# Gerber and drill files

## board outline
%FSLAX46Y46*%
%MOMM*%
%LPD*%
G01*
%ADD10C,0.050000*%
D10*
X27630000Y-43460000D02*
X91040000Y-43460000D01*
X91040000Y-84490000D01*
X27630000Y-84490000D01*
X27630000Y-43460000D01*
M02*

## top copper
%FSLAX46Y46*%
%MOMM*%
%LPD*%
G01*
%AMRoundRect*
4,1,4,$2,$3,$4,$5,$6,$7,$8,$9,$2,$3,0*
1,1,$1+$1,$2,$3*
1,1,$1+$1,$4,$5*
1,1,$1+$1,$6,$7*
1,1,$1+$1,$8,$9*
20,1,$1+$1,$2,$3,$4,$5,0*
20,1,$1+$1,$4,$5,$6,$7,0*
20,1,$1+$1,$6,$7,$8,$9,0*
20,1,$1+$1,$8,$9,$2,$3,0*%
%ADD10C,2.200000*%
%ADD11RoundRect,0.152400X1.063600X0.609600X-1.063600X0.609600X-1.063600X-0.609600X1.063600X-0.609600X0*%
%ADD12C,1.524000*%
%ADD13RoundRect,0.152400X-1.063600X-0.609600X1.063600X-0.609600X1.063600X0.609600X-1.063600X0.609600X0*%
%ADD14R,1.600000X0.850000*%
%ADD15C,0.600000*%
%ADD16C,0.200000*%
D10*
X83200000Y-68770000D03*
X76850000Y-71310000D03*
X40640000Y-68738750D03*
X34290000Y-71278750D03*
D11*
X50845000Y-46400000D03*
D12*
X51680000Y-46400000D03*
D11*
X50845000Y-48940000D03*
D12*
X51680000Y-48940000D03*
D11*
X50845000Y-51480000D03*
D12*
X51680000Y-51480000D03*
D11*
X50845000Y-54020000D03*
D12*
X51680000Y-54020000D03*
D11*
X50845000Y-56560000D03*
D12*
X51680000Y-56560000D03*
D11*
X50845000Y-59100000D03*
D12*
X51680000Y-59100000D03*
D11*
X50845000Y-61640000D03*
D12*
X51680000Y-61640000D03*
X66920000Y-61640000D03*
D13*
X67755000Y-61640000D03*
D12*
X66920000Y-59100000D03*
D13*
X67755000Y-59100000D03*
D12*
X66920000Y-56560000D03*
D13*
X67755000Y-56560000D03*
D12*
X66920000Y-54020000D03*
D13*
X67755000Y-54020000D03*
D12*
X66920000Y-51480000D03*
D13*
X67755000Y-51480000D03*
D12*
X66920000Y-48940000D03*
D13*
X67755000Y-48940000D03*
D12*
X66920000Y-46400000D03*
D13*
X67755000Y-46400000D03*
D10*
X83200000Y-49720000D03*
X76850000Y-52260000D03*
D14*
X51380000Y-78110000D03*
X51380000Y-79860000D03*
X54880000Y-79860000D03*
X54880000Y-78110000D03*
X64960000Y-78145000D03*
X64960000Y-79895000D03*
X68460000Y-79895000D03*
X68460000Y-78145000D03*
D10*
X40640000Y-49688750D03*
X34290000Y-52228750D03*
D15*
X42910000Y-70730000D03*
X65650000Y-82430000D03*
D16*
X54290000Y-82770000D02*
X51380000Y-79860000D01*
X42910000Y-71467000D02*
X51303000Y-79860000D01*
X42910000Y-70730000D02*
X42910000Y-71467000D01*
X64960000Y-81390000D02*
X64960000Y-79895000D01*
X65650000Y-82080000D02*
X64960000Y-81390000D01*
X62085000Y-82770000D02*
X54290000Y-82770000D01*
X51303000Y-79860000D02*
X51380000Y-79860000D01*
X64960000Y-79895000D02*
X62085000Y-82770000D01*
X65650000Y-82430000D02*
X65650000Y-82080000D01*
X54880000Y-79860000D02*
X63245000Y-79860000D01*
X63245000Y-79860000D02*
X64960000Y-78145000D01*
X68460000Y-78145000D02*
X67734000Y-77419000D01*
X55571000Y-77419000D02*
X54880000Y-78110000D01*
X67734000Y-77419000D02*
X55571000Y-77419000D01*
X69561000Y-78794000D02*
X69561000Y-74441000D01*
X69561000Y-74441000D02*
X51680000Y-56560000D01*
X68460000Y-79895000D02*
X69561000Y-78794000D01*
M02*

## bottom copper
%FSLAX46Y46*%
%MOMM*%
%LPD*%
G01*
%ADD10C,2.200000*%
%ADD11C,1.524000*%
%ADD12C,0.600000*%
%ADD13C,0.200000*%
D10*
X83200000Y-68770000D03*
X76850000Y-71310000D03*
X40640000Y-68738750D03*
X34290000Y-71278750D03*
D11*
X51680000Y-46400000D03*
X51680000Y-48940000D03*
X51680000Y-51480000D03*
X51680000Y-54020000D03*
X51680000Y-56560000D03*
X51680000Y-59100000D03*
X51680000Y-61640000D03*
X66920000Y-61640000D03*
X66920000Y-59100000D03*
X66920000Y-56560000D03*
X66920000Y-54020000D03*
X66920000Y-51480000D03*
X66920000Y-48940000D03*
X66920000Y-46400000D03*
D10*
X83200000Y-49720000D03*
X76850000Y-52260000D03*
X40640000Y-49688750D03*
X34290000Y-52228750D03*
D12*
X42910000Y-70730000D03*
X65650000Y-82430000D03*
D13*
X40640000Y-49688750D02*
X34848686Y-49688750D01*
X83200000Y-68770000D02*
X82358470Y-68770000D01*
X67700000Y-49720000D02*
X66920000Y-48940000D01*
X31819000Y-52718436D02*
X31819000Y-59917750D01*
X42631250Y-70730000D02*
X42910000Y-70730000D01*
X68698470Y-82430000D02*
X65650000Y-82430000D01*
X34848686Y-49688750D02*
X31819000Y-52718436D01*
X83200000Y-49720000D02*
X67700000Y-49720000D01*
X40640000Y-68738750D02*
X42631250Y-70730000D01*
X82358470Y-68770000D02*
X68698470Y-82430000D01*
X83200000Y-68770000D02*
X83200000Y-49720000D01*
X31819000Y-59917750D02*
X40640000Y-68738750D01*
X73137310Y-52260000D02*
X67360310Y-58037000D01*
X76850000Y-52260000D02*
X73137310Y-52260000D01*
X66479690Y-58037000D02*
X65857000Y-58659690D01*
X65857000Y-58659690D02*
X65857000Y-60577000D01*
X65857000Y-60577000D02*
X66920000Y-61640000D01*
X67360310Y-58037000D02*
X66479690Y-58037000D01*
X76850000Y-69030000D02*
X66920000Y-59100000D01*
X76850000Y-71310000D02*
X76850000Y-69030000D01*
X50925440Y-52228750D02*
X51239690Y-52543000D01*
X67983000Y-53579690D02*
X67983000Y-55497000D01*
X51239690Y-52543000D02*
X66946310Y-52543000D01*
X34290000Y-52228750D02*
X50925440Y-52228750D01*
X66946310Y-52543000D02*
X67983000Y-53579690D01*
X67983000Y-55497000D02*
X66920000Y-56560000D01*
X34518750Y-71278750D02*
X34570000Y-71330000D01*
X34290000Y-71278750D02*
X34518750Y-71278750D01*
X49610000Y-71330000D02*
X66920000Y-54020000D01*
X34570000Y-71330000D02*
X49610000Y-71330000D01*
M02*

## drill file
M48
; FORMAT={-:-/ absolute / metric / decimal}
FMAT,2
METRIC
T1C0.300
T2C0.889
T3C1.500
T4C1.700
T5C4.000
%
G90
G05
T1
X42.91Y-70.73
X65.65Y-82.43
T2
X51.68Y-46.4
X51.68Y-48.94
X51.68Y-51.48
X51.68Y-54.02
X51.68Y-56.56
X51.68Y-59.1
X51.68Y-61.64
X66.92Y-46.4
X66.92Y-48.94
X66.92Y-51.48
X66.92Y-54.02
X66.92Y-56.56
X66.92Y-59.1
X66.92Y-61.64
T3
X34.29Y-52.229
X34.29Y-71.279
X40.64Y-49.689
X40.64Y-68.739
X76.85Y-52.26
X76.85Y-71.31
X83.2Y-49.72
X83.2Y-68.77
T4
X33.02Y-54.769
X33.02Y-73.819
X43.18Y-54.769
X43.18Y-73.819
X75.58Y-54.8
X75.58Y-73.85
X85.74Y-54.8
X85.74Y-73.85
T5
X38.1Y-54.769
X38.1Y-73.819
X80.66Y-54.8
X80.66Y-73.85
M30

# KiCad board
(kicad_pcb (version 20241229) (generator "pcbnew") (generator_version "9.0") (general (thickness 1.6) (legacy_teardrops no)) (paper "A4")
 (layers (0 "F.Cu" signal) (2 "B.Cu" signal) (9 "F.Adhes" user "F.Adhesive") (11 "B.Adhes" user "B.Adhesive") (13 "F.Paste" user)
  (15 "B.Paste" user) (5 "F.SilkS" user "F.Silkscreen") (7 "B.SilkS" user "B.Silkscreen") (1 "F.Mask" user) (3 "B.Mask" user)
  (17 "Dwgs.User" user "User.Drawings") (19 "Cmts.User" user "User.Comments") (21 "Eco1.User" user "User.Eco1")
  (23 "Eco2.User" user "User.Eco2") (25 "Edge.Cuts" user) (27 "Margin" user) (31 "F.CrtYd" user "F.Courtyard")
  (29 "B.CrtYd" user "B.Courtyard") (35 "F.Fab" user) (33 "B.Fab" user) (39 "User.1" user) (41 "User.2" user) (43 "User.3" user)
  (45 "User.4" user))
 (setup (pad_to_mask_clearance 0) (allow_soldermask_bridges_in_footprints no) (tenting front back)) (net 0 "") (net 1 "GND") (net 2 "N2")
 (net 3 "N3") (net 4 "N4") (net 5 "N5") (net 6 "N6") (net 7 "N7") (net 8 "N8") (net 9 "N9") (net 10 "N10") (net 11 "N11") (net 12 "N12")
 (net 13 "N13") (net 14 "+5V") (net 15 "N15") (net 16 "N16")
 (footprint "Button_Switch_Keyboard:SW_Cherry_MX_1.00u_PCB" (layer "F.Cu") (at 83.2 68.77)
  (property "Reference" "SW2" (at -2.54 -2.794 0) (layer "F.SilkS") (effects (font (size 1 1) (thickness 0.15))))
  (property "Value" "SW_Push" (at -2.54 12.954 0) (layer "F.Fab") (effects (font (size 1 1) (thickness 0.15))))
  (pad "" np_thru_hole circle (at -7.62 5.08) (size 1.7 1.7) (drill 1.7) (layers "*.Cu" "*.Mask"))
  (pad "" np_thru_hole circle (at -2.54 5.08) (size 4 4) (drill 4) (layers "*.Cu" "*.Mask"))
  (pad "" np_thru_hole circle (at 2.54 5.08) (size 1.7 1.7) (drill 1.7) (layers "*.Cu" "*.Mask"))
  (pad "1" thru_hole circle (at 0 0) (size 2.2 2.2) (drill 1.5) (layers "*.Cu" "*.Mask") (remove_unused_layers no) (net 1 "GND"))
  (pad "2" thru_hole circle (at -6.35 2.54) (size 2.2 2.2) (drill 1.5) (layers "*.Cu" "*.Mask") (remove_unused_layers no) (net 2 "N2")))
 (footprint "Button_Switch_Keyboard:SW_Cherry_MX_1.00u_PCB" (layer "F.Cu") (at 40.64 68.73875)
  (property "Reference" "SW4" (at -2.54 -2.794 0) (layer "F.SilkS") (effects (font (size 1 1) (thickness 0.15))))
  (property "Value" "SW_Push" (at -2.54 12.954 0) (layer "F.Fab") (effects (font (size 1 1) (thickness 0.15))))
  (pad "" np_thru_hole circle (at -7.62 5.08) (size 1.7 1.7) (drill 1.7) (layers "*.Cu" "*.Mask"))
  (pad "" np_thru_hole circle (at -2.54 5.08) (size 4 4) (drill 4) (layers "*.Cu" "*.Mask"))
  (pad "" np_thru_hole circle (at 2.54 5.08) (size 1.7 1.7) (drill 1.7) (layers "*.Cu" "*.Mask"))
  (pad "1" thru_hole circle (at 0 0) (size 2.2 2.2) (drill 1.5) (layers "*.Cu" "*.Mask") (remove_unused_layers no) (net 1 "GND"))
  (pad "2" thru_hole circle (at -6.35 2.54) (size 2.2 2.2) (drill 1.5) (layers "*.Cu" "*.Mask") (remove_unused_layers no) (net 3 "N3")))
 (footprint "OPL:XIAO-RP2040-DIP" (layer "F.Cu") (at 59.3 54.02)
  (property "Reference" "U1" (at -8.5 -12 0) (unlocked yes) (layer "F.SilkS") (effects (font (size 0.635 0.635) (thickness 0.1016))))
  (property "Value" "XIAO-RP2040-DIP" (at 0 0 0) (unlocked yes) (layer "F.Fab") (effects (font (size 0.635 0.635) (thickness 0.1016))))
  (pad "1" smd roundrect (at -8.455 -7.62 180) (size 2.432 1.524) (layers "F.Cu" "F.Mask") (roundrect_rratio 0.1) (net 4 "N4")
   (thermal_bridge_angle 45))
  (pad "1" thru_hole circle (at -7.62 -7.62 180) (size 1.524 1.524) (drill 0.889) (layers "*.Cu" "*.Mask") (remove_unused_layers no)
   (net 4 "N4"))
  (pad "2" smd roundrect (at -8.455 -5.08 180) (size 2.432 1.524) (layers "F.Cu" "F.Mask") (roundrect_rratio 0.1) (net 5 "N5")
   (thermal_bridge_angle 45))
  (pad "2" thru_hole circle (at -7.62 -5.08 180) (size 1.524 1.524) (drill 0.889) (layers "*.Cu" "*.Mask") (remove_unused_layers no)
   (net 5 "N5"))
  (pad "3" smd roundrect (at -8.455 -2.54 180) (size 2.432 1.524) (layers "F.Cu" "F.Mask") (roundrect_rratio 0.1) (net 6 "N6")
   (thermal_bridge_angle 45))
  (pad "3" thru_hole circle (at -7.62 -2.54 180) (size 1.524 1.524) (drill 0.889) (layers "*.Cu" "*.Mask") (remove_unused_layers no)
   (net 6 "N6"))
  (pad "4" smd roundrect (at -8.455 0 180) (size 2.432 1.524) (layers "F.Cu" "F.Mask") (roundrect_rratio 0.1) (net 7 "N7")
   (thermal_bridge_angle 45))
  (pad "4" thru_hole circle (at -7.62 0 180) (size 1.524 1.524) (drill 0.889) (layers "*.Cu" "*.Mask") (remove_unused_layers no)
   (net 7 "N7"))
  (pad "5" smd roundrect (at -8.455 2.54 180) (size 2.432 1.524) (layers "F.Cu" "F.Mask") (roundrect_rratio 0.1) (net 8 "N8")
   (thermal_bridge_angle 45))
  (pad "5" thru_hole circle (at -7.62 2.54 180) (size 1.524 1.524) (drill 0.889) (layers "*.Cu" "*.Mask") (remove_unused_layers no)
   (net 8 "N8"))
  (pad "6" smd roundrect (at -8.455 5.08 180) (size 2.432 1.524) (layers "F.Cu" "F.Mask") (roundrect_rratio 0.1) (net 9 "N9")
   (thermal_bridge_angle 45))
  (pad "6" thru_hole circle (at -7.62 5.08 180) (size 1.524 1.524) (drill 0.889) (layers "*.Cu" "*.Mask") (remove_unused_layers no)
   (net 9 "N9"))
  (pad "7" smd roundrect (at -8.455 7.62 180) (size 2.432 1.524) (layers "F.Cu" "F.Mask") (roundrect_rratio 0.1) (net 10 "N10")
   (thermal_bridge_angle 45))
  (pad "7" thru_hole circle (at -7.62 7.62 180) (size 1.524 1.524) (drill 0.889) (layers "*.Cu" "*.Mask") (remove_unused_layers no)
   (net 10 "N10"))
  (pad "8" thru_hole circle (at 7.62 7.62) (size 1.524 1.524) (drill 0.889) (layers "*.Cu" "*.Mask") (remove_unused_layers no)
   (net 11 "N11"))
  (pad "8" smd roundrect (at 8.455 7.62) (size 2.432 1.524) (layers "F.Cu" "F.Mask") (roundrect_rratio 0.1) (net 11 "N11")
   (thermal_bridge_angle 45))
  (pad "9" thru_hole circle (at 7.62 5.08) (size 1.524 1.524) (drill 0.889) (layers "*.Cu" "*.Mask") (remove_unused_layers no) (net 2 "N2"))
  (pad "9" smd roundrect (at 8.455 5.08) (size 2.432 1.524) (layers "F.Cu" "F.Mask") (roundrect_rratio 0.1) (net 2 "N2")
   (thermal_bridge_angle 45))
  (pad "10" thru_hole circle (at 7.62 2.54) (size 1.524 1.524) (drill 0.889) (layers "*.Cu" "*.Mask") (remove_unused_layers no)
   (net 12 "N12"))
  (pad "10" smd roundrect (at 8.455 2.54) (size 2.432 1.524) (layers "F.Cu" "F.Mask") (roundrect_rratio 0.1) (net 12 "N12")
   (thermal_bridge_angle 45))
  (pad "11" thru_hole circle (at 7.62 0) (size 1.524 1.524) (drill 0.889) (layers "*.Cu" "*.Mask") (remove_unused_layers no) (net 3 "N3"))
  (pad "11" smd roundrect (at 8.455 0) (size 2.432 1.524) (layers "F.Cu" "F.Mask") (roundrect_rratio 0.1) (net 3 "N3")
   (thermal_bridge_angle 45))
  (pad "12" thru_hole circle (at 7.62 -2.54) (size 1.524 1.524) (drill 0.889) (layers "*.Cu" "*.Mask") (remove_unused_layers no)
   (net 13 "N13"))
  (pad "12" smd roundrect (at 8.455 -2.54) (size 2.432 1.524) (layers "F.Cu" "F.Mask") (roundrect_rratio 0.1) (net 13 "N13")
   (thermal_bridge_angle 45))
  (pad "13" thru_hole circle (at 7.62 -5.08) (size 1.524 1.524) (drill 0.889) (layers "*.Cu" "*.Mask") (remove_unused_layers no)
   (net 1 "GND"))
  (pad "13" smd roundrect (at 8.455 -5.08) (size 2.432 1.524) (layers "F.Cu" "F.Mask") (roundrect_rratio 0.1) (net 1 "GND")
   (thermal_bridge_angle 45))
  (pad "14" thru_hole circle (at 7.62 -7.62) (size 1.524 1.524) (drill 0.889) (layers "*.Cu" "*.Mask") (remove_unused_layers no)
   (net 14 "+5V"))
  (pad "14" smd roundrect (at 8.455 -7.62) (size 2.432 1.524) (layers "F.Cu" "F.Mask") (roundrect_rratio 0.1) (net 14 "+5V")
   (thermal_bridge_angle 45)))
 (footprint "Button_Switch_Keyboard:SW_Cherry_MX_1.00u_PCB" (layer "F.Cu") (at 83.2 49.72)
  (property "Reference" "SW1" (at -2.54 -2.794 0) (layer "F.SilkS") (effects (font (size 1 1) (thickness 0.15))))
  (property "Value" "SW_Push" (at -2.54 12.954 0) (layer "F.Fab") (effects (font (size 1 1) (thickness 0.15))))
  (pad "" np_thru_hole circle (at -7.62 5.08) (size 1.7 1.7) (drill 1.7) (layers "*.Cu" "*.Mask"))
  (pad "" np_thru_hole circle (at -2.54 5.08) (size 4 4) (drill 4) (layers "*.Cu" "*.Mask"))
  (pad "" np_thru_hole circle (at 2.54 5.08) (size 1.7 1.7) (drill 1.7) (layers "*.Cu" "*.Mask"))
  (pad "1" thru_hole circle (at 0 0) (size 2.2 2.2) (drill 1.5) (layers "*.Cu" "*.Mask") (remove_unused_layers no) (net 1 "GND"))
  (pad "2" thru_hole circle (at -6.35 2.54) (size 2.2 2.2) (drill 1.5) (layers "*.Cu" "*.Mask") (remove_unused_layers no) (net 11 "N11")))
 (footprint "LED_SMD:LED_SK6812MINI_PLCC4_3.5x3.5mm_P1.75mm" (layer "F.Cu") (at 53.13 78.985)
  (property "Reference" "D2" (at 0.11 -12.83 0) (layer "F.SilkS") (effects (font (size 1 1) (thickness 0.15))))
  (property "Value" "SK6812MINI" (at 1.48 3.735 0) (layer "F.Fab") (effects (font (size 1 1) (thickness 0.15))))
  (pad "1" smd rect (at -1.75 -0.875) (size 1.6 0.85) (layers "F.Cu" "F.Mask" "F.Paste") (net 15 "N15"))
  (pad "2" smd rect (at -1.75 0.875) (size 1.6 0.85) (layers "F.Cu" "F.Mask" "F.Paste") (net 1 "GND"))
  (pad "3" smd rect (at 1.75 0.875) (size 1.6 0.85) (layers "F.Cu" "F.Mask" "F.Paste") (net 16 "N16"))
  (pad "4" smd rect (at 1.75 -0.875) (size 1.6 0.85) (layers "F.Cu" "F.Mask" "F.Paste") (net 14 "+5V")))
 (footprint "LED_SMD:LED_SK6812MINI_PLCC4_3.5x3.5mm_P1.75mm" (layer "F.Cu") (at 66.71 79.02)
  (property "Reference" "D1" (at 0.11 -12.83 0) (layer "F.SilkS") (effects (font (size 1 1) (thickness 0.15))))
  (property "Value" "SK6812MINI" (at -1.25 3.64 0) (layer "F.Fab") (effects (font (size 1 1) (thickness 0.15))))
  (pad "1" smd rect (at -1.75 -0.875) (size 1.6 0.85) (layers "F.Cu" "F.Mask" "F.Paste") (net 16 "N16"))
  (pad "2" smd rect (at -1.75 0.875) (size 1.6 0.85) (layers "F.Cu" "F.Mask" "F.Paste") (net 1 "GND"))
  (pad "3" smd rect (at 1.75 0.875) (size 1.6 0.85) (layers "F.Cu" "F.Mask" "F.Paste") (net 8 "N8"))
  (pad "4" smd rect (at 1.75 -0.875) (size 1.6 0.85) (layers "F.Cu" "F.Mask" "F.Paste") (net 14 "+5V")))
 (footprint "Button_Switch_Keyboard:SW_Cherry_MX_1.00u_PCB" (layer "F.Cu") (at 40.64 49.68875)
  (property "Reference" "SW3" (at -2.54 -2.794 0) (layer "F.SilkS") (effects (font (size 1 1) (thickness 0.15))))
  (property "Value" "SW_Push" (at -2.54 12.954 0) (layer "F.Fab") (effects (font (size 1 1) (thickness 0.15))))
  (pad "" np_thru_hole circle (at -7.62 5.08) (size 1.7 1.7) (drill 1.7) (layers "*.Cu" "*.Mask"))
  (pad "" np_thru_hole circle (at -2.54 5.08) (size 4 4) (drill 4) (layers "*.Cu" "*.Mask"))
  (pad "" np_thru_hole circle (at 2.54 5.08) (size 1.7 1.7) (drill 1.7) (layers "*.Cu" "*.Mask"))
  (pad "1" thru_hole circle (at 0 0) (size 2.2 2.2) (drill 1.5) (layers "*.Cu" "*.Mask") (remove_unused_layers no) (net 1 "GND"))
  (pad "2" thru_hole circle (at -6.35 2.54) (size 2.2 2.2) (drill 1.5) (layers "*.Cu" "*.Mask") (remove_unused_layers no) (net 12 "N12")))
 (gr_rect (start 27.63 43.46) (end 91.04 84.49) (stroke (width 0.05) (type default)) (fill no) (layer "Edge.Cuts"))
 (segment (start 54.29 82.77) (end 51.38 79.86) (width 0.2) (layer "F.Cu") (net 1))
 (segment (start 42.91 71.467) (end 51.303 79.86) (width 0.2) (layer "F.Cu") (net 1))
 (segment (start 42.91 70.73) (end 42.91 71.467) (width 0.2) (layer "F.Cu") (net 1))
 (segment (start 64.96 81.39) (end 64.96 79.895) (width 0.2) (layer "F.Cu") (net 1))
 (segment (start 65.65 82.08) (end 64.96 81.39) (width 0.2) (layer "F.Cu") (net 1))
 (segment (start 62.085 82.77) (end 54.29 82.77) (width 0.2) (layer "F.Cu") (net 1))
 (segment (start 51.303 79.86) (end 51.38 79.86) (width 0.2) (layer "F.Cu") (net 1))
 (segment (start 64.96 79.895) (end 62.085 82.77) (width 0.2) (layer "F.Cu") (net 1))
 (segment (start 65.65 82.43) (end 65.65 82.08) (width 0.2) (layer "F.Cu") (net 1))
 (via (at 42.91 70.73) (size 0.6) (drill 0.3) (layers "F.Cu" "B.Cu") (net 1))
 (via (at 65.65 82.43) (size 0.6) (drill 0.3) (layers "F.Cu" "B.Cu") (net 1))
 (segment (start 40.64 49.68875) (end 34.848686 49.68875) (width 0.2) (layer "B.Cu") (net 1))
 (segment (start 83.2 68.77) (end 82.35847 68.77) (width 0.2) (layer "B.Cu") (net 1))
 (segment (start 67.7 49.72) (end 66.92 48.94) (width 0.2) (layer "B.Cu") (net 1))
 (segment (start 31.819 52.718436) (end 31.819 59.91775) (width 0.2) (layer "B.Cu") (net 1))
 (segment (start 42.63125 70.73) (end 42.91 70.73) (width 0.2) (layer "B.Cu") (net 1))
 (segment (start 68.69847 82.43) (end 65.65 82.43) (width 0.2) (layer "B.Cu") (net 1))
 (segment (start 34.848686 49.68875) (end 31.819 52.718436) (width 0.2) (layer "B.Cu") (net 1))
 (segment (start 83.2 49.72) (end 67.7 49.72) (width 0.2) (layer "B.Cu") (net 1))
 (segment (start 40.64 68.73875) (end 42.63125 70.73) (width 0.2) (layer "B.Cu") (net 1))
 (segment (start 82.35847 68.77) (end 68.69847 82.43) (width 0.2) (layer "B.Cu") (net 1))
 (segment (start 83.2 68.77) (end 83.2 49.72) (width 0.2) (layer "B.Cu") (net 1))
 (segment (start 31.819 59.91775) (end 40.64 68.73875) (width 0.2) (layer "B.Cu") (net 1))
 (segment (start 54.88 79.86) (end 63.245 79.86) (width 0.2) (layer "F.Cu") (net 16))
 (segment (start 63.245 79.86) (end 64.96 78.145) (width 0.2) (layer "F.Cu") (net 16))
 (segment (start 68.46 78.145) (end 67.734 77.419) (width 0.2) (layer "F.Cu") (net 14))
 (segment (start 55.571 77.419) (end 54.88 78.11) (width 0.2) (layer "F.Cu") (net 14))
 (segment (start 67.734 77.419) (end 55.571 77.419) (width 0.2) (layer "F.Cu") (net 14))
 (segment (start 69.561 78.794) (end 69.561 74.441) (width 0.2) (layer "F.Cu") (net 8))
 (segment (start 69.561 74.441) (end 51.68 56.56) (width 0.2) (layer "F.Cu") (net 8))
 (segment (start 68.46 79.895) (end 69.561 78.794) (width 0.2) (layer "F.Cu") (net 8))
 (segment (start 73.13731 52.26) (end 67.36031 58.037) (width 0.2) (layer "B.Cu") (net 11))
 (segment (start 76.85 52.26) (end 73.13731 52.26) (width 0.2) (layer "B.Cu") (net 11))
 (segment (start 66.47969 58.037) (end 65.857 58.65969) (width 0.2) (layer "B.Cu") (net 11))
 (segment (start 65.857 58.65969) (end 65.857 60.577) (width 0.2) (layer "B.Cu") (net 11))
 (segment (start 65.857 60.577) (end 66.92 61.64) (width 0.2) (layer "B.Cu") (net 11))
 (segment (start 67.36031 58.037) (end 66.47969 58.037) (width 0.2) (layer "B.Cu") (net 11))
 (segment (start 76.85 69.03) (end 66.92 59.1) (width 0.2) (layer "B.Cu") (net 2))
 (segment (start 76.85 71.31) (end 76.85 69.03) (width 0.2) (layer "B.Cu") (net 2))
 (segment (start 50.92544 52.22875) (end 51.23969 52.543) (width 0.2) (layer "B.Cu") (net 12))
 (segment (start 67.983 53.57969) (end 67.983 55.497) (width 0.2) (layer "B.Cu") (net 12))
 (segment (start 51.23969 52.543) (end 66.94631 52.543) (width 0.2) (layer "B.Cu") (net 12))
 (segment (start 34.29 52.22875) (end 50.92544 52.22875) (width 0.2) (layer "B.Cu") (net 12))
 (segment (start 66.94631 52.543) (end 67.983 53.57969) (width 0.2) (layer "B.Cu") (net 12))
 (segment (start 67.983 55.497) (end 66.92 56.56) (width 0.2) (layer "B.Cu") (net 12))
 (segment (start 34.51875 71.27875) (end 34.57 71.33) (width 0.2) (layer "B.Cu") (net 3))
 (segment (start 34.29 71.27875) (end 34.51875 71.27875) (width 0.2) (layer "B.Cu") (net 3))
 (segment (start 49.61 71.33) (end 66.92 54.02) (width 0.2) (layer "B.Cu") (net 3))
 (segment (start 34.57 71.33) (end 49.61 71.33) (width 0.2) (layer "B.Cu") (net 3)))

